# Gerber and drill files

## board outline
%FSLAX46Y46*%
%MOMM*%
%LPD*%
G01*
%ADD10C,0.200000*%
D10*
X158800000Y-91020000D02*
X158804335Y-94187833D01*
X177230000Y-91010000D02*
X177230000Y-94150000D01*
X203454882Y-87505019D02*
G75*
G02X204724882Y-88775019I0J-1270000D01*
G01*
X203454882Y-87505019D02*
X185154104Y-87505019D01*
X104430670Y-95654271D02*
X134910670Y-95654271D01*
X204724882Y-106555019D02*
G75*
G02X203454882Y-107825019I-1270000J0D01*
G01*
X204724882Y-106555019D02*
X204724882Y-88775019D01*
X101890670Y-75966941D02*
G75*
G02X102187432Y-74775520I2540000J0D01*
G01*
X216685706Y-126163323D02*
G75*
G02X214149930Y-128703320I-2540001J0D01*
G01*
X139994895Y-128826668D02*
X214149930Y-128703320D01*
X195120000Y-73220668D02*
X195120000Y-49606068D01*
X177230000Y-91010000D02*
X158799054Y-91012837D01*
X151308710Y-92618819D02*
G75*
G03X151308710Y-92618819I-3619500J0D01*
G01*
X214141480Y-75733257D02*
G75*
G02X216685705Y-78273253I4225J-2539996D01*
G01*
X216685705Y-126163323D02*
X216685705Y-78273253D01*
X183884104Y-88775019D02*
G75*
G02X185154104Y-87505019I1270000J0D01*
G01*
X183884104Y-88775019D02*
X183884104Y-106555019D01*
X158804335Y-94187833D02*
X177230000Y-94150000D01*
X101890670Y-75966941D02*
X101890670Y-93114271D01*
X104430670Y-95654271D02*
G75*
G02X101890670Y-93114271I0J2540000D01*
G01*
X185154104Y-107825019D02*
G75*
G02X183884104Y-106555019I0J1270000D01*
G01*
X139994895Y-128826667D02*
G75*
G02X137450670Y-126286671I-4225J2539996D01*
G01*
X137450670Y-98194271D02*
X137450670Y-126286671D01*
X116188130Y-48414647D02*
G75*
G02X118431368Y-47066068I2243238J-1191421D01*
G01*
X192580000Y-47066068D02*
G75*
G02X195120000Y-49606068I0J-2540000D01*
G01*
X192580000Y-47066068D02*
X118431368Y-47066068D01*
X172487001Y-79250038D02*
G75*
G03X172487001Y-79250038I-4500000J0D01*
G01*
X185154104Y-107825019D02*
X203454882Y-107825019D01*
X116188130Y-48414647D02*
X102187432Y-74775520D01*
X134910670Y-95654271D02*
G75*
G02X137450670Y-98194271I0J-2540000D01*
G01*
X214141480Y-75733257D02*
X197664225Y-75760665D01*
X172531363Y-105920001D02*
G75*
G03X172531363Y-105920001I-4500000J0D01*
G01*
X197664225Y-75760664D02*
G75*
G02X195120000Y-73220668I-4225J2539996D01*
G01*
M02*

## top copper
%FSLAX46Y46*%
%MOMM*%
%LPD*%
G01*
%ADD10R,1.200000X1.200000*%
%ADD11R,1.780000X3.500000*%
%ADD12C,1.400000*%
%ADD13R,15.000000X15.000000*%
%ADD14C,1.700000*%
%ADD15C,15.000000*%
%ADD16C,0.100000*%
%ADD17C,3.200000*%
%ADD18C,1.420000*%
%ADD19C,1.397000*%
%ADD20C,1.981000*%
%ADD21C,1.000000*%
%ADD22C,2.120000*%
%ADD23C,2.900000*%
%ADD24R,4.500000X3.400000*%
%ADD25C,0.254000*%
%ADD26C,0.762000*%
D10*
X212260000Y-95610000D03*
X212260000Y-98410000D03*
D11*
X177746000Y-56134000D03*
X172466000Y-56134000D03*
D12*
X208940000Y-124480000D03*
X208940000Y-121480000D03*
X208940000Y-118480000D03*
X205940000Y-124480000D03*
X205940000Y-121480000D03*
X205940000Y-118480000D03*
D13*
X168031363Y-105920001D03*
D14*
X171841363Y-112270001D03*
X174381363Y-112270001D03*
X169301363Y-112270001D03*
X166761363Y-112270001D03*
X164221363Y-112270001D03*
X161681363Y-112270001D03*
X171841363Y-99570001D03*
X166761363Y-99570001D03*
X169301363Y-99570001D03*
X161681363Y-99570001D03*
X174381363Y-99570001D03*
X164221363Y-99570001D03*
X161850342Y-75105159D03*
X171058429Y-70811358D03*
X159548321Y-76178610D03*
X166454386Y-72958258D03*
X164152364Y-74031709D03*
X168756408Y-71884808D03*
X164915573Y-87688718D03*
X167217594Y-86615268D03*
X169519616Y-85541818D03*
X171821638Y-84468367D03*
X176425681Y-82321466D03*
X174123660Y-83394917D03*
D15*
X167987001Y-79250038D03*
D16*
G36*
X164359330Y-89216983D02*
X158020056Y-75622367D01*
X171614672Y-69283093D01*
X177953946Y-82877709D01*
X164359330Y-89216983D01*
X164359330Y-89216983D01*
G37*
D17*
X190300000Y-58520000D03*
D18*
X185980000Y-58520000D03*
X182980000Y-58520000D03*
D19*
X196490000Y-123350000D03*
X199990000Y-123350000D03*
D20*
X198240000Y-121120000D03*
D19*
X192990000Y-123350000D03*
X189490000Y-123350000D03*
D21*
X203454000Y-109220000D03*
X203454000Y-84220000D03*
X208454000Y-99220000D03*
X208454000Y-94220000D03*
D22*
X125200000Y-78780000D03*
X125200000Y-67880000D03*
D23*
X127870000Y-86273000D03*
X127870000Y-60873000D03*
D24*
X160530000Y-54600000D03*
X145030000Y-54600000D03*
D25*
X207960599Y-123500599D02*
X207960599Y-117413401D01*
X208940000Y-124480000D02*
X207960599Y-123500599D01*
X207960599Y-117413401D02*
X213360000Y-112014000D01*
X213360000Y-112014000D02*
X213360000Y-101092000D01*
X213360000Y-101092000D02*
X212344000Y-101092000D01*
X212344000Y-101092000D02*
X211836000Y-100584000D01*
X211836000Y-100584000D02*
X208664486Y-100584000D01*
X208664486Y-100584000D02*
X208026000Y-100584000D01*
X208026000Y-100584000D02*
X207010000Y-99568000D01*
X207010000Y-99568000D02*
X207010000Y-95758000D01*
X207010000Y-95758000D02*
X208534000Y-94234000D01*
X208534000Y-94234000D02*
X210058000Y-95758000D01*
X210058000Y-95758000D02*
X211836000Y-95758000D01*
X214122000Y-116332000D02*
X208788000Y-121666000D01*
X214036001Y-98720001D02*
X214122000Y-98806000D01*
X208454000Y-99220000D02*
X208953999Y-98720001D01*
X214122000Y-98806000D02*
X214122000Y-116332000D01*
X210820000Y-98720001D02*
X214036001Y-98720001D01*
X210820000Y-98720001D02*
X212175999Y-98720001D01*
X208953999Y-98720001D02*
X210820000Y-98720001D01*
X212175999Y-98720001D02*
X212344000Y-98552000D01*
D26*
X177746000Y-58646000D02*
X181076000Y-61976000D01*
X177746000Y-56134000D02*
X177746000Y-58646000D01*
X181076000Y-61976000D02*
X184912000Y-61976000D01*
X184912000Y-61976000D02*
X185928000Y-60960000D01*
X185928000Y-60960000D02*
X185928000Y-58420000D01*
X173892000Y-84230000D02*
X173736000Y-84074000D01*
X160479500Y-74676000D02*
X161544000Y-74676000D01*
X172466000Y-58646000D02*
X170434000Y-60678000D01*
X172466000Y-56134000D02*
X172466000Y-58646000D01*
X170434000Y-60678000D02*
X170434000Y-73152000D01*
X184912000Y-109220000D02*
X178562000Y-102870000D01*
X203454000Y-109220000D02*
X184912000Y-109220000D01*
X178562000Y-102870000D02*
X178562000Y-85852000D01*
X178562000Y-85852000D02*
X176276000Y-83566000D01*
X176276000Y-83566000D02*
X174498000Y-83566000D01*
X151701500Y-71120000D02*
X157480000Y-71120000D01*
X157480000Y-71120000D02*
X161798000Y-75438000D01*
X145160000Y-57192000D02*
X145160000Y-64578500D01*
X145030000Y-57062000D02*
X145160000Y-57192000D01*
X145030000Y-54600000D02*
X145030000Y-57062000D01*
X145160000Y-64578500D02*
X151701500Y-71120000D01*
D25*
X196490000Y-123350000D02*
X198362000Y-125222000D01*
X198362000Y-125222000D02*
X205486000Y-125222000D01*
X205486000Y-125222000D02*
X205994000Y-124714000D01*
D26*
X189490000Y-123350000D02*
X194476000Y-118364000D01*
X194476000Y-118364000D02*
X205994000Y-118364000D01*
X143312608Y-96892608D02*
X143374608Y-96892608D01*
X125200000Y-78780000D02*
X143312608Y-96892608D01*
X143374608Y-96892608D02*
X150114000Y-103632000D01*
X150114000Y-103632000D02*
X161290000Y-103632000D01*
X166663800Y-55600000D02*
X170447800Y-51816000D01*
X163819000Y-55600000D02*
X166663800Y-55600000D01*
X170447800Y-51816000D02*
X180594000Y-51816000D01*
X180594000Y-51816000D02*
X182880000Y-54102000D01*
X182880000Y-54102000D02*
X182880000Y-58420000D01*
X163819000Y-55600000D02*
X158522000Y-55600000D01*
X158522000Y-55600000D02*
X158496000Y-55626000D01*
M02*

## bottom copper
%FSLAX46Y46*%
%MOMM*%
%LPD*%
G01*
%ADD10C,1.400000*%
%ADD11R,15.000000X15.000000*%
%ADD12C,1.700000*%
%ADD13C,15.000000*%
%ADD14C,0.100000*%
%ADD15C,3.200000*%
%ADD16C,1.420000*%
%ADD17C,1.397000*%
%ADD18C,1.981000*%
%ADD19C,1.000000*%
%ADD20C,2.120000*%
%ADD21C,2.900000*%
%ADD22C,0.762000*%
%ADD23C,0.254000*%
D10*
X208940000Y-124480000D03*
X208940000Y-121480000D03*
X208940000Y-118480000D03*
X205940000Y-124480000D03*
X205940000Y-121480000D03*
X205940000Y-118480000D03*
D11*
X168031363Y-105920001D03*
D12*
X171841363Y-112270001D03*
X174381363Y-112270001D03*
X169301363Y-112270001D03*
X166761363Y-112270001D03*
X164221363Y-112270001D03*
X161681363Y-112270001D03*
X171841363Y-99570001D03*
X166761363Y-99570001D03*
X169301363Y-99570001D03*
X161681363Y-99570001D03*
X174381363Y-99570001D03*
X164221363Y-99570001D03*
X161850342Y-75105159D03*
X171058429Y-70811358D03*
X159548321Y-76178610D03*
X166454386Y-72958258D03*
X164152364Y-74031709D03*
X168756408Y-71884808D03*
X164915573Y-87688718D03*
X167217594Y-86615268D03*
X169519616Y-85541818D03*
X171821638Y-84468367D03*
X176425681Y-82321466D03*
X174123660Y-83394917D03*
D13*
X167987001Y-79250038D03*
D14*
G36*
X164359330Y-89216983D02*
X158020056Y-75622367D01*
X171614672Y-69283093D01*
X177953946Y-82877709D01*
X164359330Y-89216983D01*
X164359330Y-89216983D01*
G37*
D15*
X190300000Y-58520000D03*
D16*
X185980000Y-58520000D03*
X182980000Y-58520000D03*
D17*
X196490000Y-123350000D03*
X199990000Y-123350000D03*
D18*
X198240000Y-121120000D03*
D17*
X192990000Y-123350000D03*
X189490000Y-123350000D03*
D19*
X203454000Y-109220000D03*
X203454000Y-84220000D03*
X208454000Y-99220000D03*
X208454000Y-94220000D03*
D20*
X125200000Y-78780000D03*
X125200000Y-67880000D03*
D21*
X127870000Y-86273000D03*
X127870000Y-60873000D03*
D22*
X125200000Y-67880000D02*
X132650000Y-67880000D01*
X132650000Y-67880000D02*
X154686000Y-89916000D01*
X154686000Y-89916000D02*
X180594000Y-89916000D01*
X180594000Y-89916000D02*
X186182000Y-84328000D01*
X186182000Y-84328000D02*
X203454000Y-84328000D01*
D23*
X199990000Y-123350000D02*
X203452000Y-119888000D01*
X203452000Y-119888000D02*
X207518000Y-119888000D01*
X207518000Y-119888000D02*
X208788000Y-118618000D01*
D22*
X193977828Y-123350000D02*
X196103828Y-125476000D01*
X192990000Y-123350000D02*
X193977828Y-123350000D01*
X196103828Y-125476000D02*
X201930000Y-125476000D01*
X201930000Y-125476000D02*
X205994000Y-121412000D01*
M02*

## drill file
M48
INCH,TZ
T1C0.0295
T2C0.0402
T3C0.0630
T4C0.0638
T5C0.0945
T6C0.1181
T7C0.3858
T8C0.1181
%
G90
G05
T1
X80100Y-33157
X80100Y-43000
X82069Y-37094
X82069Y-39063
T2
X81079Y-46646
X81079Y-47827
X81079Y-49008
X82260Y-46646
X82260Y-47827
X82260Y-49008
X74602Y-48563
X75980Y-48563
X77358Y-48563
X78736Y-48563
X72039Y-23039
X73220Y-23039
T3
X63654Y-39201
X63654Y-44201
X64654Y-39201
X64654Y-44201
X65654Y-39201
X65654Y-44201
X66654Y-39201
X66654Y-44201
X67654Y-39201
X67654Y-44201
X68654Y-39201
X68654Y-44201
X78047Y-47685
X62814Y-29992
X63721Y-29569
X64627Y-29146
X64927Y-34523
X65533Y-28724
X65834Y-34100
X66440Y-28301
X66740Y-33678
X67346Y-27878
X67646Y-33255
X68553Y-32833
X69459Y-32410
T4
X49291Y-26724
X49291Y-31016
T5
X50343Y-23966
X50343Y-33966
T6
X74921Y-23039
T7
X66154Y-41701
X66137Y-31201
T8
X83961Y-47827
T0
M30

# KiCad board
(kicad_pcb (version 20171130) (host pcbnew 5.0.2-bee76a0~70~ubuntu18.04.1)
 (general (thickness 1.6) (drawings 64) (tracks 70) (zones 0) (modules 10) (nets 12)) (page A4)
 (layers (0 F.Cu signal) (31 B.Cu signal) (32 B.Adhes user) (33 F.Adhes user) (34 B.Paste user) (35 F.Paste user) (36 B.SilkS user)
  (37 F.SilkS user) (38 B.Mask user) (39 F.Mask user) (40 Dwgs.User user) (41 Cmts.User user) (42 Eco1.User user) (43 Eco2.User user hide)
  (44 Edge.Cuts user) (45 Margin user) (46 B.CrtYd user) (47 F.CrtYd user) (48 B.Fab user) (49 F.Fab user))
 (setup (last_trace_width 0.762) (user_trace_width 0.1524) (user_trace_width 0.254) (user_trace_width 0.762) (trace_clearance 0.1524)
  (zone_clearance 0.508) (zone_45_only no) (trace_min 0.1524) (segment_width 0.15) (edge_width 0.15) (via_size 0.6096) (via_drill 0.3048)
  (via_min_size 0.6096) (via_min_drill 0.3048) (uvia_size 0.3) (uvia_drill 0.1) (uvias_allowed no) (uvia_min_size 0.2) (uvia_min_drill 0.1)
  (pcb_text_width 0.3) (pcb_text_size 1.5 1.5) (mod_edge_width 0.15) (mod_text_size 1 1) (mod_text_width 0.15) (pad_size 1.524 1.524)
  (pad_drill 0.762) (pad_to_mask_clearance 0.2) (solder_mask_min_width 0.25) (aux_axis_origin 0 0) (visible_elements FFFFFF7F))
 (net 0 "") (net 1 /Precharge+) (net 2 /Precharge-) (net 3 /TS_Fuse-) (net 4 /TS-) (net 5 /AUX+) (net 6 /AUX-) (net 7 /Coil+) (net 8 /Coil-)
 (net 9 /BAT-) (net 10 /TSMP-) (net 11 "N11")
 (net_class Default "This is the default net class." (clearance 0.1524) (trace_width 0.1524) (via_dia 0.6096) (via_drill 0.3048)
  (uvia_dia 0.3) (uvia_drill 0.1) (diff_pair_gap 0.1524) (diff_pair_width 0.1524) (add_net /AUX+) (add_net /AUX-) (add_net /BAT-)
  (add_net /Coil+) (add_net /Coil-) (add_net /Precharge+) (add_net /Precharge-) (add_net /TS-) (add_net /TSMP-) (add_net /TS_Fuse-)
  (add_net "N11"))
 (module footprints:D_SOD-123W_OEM (layer F.Cu) (at 212.26 97.01 270)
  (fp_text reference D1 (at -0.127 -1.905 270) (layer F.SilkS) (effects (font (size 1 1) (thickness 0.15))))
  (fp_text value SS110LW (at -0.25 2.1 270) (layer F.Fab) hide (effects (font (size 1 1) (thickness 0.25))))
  (pad 1 smd rect (at -1.4 0 270) (size 1.2 1.2) (layers F.Cu F.Paste F.Mask) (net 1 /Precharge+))
  (pad 2 smd rect (at 1.4 0 270) (size 1.2 1.2) (layers F.Cu F.Paste F.Mask) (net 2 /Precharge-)))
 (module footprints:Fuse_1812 (layer F.Cu) (at 172.466 56.134)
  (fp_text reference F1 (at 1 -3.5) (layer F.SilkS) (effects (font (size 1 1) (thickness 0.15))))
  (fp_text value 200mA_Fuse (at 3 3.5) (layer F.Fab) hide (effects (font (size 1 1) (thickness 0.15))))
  (pad 2 smd rect (at 5.28 0) (size 1.78 3.5) (layers F.Cu F.Paste F.Mask) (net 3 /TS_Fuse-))
  (pad 1 smd rect (at 0 0) (size 1.78 3.5) (layers F.Cu F.Paste F.Mask) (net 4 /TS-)))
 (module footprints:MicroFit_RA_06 (layer B.Cu) (at 213.26 121.48 90)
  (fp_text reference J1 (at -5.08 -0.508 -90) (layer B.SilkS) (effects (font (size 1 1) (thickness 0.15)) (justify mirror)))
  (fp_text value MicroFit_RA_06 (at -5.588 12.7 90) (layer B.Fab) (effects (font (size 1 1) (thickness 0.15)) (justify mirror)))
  (pad "" np_thru_hole circle (at 0 0 270) (size 3 3) (drill 3) (layers *.Cu *.Mask))
  (pad 1 thru_hole circle (at -3 -4.32 270) (size 1.4 1.4) (drill 1.02) (layers *.Cu *.Mask) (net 1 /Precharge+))
  (pad 2 thru_hole circle (at 0 -4.32 270) (size 1.4 1.4) (drill 1.02) (layers *.Cu *.Mask) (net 2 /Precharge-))
  (pad 3 thru_hole circle (at 3 -4.32 270) (size 1.4 1.4) (drill 1.02) (layers *.Cu *.Mask) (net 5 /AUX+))
  (pad 4 thru_hole circle (at -3 -7.32 270) (size 1.4 1.4) (drill 1.02) (layers *.Cu *.Mask) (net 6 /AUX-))
  (pad 5 thru_hole circle (at 0 -7.32 270) (size 1.4 1.4) (drill 1.02) (layers *.Cu *.Mask) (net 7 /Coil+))
  (pad 6 thru_hole circle (at 3 -7.32 270) (size 1.4 1.4) (drill 1.02) (layers *.Cu *.Mask) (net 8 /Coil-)))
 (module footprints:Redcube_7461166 (layer F.Cu) (at 168.031363 105.920001)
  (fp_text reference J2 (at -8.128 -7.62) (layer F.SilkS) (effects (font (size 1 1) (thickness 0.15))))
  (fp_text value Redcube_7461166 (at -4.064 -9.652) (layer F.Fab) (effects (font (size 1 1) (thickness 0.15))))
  (pad 1 thru_hole rect (at 0 0) (size 15 15) (drill 9.8) (layers *.Cu *.Mask) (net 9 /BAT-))
  (pad 1 thru_hole circle (at 3.81 6.35) (size 1.7 1.7) (drill 1.6) (layers *.Cu *.Mask) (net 9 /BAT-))
  (pad 1 thru_hole circle (at 6.35 6.35) (size 1.7 1.7) (drill 1.6) (layers *.Cu *.Mask) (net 9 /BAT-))
  (pad 1 thru_hole circle (at 1.27 6.35) (size 1.7 1.7) (drill 1.6) (layers *.Cu *.Mask) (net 9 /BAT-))
  (pad 1 thru_hole circle (at -1.27 6.35) (size 1.7 1.7) (drill 1.6) (layers *.Cu *.Mask) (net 9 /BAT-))
  (pad 1 thru_hole circle (at -3.81 6.35) (size 1.7 1.7) (drill 1.6) (layers *.Cu *.Mask) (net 9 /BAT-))
  (pad 1 thru_hole circle (at -6.35 6.35) (size 1.7 1.7) (drill 1.6) (layers *.Cu *.Mask) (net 9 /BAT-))
  (pad 1 thru_hole circle (at 3.81 -6.35) (size 1.7 1.7) (drill 1.6) (layers *.Cu *.Mask) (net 9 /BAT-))
  (pad 1 thru_hole circle (at -1.27 -6.35) (size 1.7 1.7) (drill 1.6) (layers *.Cu *.Mask) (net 9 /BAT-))
  (pad 1 thru_hole circle (at 1.27 -6.35) (size 1.7 1.7) (drill 1.6) (layers *.Cu *.Mask) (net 9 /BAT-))
  (pad 1 thru_hole circle (at -6.35 -6.35) (size 1.7 1.7) (drill 1.6) (layers *.Cu *.Mask) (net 9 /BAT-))
  (pad 1 thru_hole circle (at 6.35 -6.35) (size 1.7 1.7) (drill 1.6) (layers *.Cu *.Mask) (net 9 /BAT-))
  (pad 1 thru_hole circle (at -3.81 -6.35) (size 1.7 1.7) (drill 1.6) (layers *.Cu *.Mask) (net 9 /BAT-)))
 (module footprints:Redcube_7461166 (layer F.Cu) (at 167.987001 79.250038 25)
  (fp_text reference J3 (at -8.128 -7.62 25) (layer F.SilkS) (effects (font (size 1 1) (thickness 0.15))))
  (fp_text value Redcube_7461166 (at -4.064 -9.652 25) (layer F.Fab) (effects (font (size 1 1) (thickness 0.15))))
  (pad 1 thru_hole circle (at -3.81 -6.35 25) (size 1.7 1.7) (drill 1.6) (layers *.Cu *.Mask) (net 4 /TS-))
  (pad 1 thru_hole circle (at 6.349999 -6.35 25) (size 1.7 1.7) (drill 1.6) (layers *.Cu *.Mask) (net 4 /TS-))
  (pad 1 thru_hole circle (at -6.35 -6.349999 25) (size 1.7 1.7) (drill 1.6) (layers *.Cu *.Mask) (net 4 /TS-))
  (pad 1 thru_hole circle (at 1.27 -6.35 25) (size 1.7 1.7) (drill 1.6) (layers *.Cu *.Mask) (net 4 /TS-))
  (pad 1 thru_hole circle (at -1.27 -6.35 25) (size 1.7 1.7) (drill 1.6) (layers *.Cu *.Mask) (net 4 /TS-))
  (pad 1 thru_hole circle (at 3.81 -6.35 25) (size 1.7 1.7) (drill 1.6) (layers *.Cu *.Mask) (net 4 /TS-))
  (pad 1 thru_hole circle (at -6.349999 6.35 25) (size 1.7 1.7) (drill 1.6) (layers *.Cu *.Mask) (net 4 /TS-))
  (pad 1 thru_hole circle (at -3.81 6.35 25) (size 1.7 1.7) (drill 1.6) (layers *.Cu *.Mask) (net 4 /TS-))
  (pad 1 thru_hole circle (at -1.27 6.35 25) (size 1.7 1.7) (drill 1.6) (layers *.Cu *.Mask) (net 4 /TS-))
  (pad 1 thru_hole circle (at 1.27 6.35 25) (size 1.7 1.7) (drill 1.6) (layers *.Cu *.Mask) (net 4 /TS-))
  (pad 1 thru_hole circle (at 6.35 6.349999 25) (size 1.7 1.7) (drill 1.6) (layers *.Cu *.Mask) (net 4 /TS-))
  (pad 1 thru_hole circle (at 3.81 6.35 25) (size 1.7 1.7) (drill 1.6) (layers *.Cu *.Mask) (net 4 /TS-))
  (pad 1 thru_hole rect (at 0 0 25) (size 15 15) (drill 9.8) (layers *.Cu *.Mask) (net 4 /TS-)))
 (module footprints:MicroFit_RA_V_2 (layer B.Cu) (at 190.3 58.52 90)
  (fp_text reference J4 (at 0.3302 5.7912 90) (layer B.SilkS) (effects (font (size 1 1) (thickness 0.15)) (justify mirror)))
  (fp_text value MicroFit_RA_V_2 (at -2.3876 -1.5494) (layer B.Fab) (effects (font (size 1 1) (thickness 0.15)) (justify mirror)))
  (pad "" thru_hole circle (at 0 0 90) (size 3.2 3.2) (drill 3) (layers *.Cu *.Mask))
  (pad 1 thru_hole circle (at 0 -4.32 90) (size 1.42 1.42) (drill 1.02) (layers *.Cu *.Mask) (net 3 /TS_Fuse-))
  (pad 2 thru_hole circle (at 0 -7.32 90) (size 1.42 1.42) (drill 1.02) (layers *.Cu *.Mask) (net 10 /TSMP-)))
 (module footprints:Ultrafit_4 (layer F.Cu) (at 194.74 123.35 90)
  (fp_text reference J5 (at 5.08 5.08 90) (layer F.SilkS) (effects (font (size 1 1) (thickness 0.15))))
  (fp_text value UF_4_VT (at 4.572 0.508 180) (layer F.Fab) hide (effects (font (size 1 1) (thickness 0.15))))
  (pad 2 thru_hole circle (at 0 1.75 90) (size 1.397 1.397) (drill 1.02) (layers *.Cu *.Mask) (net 6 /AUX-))
  (pad 1 thru_hole circle (at 0 5.25 90) (size 1.397 1.397) (drill 1.02) (layers *.Cu *.Mask) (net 5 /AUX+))
  (pad "" thru_hole circle (at 2.23 3.5 90) (size 1.981 1.981) (drill 1.6) (layers *.Cu *.Mask))
  (pad 3 thru_hole circle (at 0 -1.75 270) (size 1.397 1.397) (drill 1.02) (layers *.Cu *.Mask) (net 7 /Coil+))
  (pad 4 thru_hole circle (at 0 -5.25 270) (size 1.397 1.397) (drill 1.02) (layers *.Cu *.Mask) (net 8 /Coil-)))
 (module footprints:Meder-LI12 (layer B.Cu) (at 203.454 109.22 90)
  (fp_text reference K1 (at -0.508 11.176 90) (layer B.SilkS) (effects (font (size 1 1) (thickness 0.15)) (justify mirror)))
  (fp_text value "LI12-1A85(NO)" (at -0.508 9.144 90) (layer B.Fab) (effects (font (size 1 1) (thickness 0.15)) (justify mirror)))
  (pad 1 thru_hole circle (at 0 0 90) (size 1 1) (drill 0.75) (layers *.Cu *.Mask) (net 4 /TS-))
  (pad 2 thru_hole circle (at 25 0 90) (size 1 1) (drill 0.75) (layers *.Cu *.Mask) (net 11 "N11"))
  (pad 3 thru_hole circle (at 10 5 90) (size 1 1) (drill 0.75) (layers *.Cu *.Mask) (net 2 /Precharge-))
  (pad 4 thru_hole circle (at 15 5 90) (size 1 1) (drill 0.75) (layers *.Cu *.Mask) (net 1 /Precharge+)))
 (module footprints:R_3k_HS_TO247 (layer B.Cu) (at 125.2 78.78 90)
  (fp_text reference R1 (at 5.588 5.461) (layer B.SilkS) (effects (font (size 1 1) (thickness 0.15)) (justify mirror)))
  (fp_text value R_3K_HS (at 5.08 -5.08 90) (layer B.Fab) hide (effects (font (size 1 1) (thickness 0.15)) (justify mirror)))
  (pad 1 thru_hole circle (at 0 0 90) (size 2.12 2.12) (drill 1.62) (layers *.Cu *.Mask) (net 9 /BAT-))
  (pad 2 thru_hole circle (at 10.9 0 90) (size 2.12 2.12) (drill 1.62) (layers *.Cu *.Mask) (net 11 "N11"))
  (pad 4 thru_hole circle (at -7.493 2.67 90) (size 2.9 2.9) (drill 2.4) (layers *.Cu *.Mask))
  (pad 5 thru_hole circle (at 17.907 2.67 90) (size 2.9 2.9) (drill 2.4) (layers *.Cu *.Mask)))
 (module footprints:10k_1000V (layer F.Cu) (at 160.53 54.6 180)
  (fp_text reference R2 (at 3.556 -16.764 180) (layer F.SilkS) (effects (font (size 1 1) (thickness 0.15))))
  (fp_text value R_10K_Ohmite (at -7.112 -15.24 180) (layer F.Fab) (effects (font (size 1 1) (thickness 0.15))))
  (pad 1 smd rect (at 0 0 180) (size 4.5 3.4) (layers F.Cu F.Paste F.Mask) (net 10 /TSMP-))
  (pad 2 smd rect (at 15.5 0 180) (size 4.5 3.4) (layers F.Cu F.Paste F.Mask) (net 4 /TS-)))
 (gr_line (start 158.8 91.02) (end 158.804335 94.187833) (layer Edge.Cuts) (width 0.2))
 (gr_line (start 177.23 91.01) (end 177.23 94.15) (layer Edge.Cuts) (width 0.2))
 (gr_arc (start 203.454882 88.775019) (end 204.724882 88.775019) (angle -90) (layer Edge.Cuts) (width 0.2))
 (gr_line (start 203.454882 87.505019) (end 185.154104 87.505019) (layer Edge.Cuts) (width 0.2))
 (gr_line (start 104.43067 95.654271) (end 134.91067 95.654271) (layer Edge.Cuts) (width 0.2))
 (gr_arc (start 203.454882 106.555019) (end 203.454882 107.825019) (angle -90) (layer Edge.Cuts) (width 0.2))
 (gr_line (start 204.724882 106.555019) (end 204.724882 88.775019) (layer Edge.Cuts) (width 0.2))
 (gr_arc (start 104.43067 75.966941) (end 102.187432 74.77552) (angle -27.9735142) (layer Edge.Cuts) (width 0.2))
 (gr_arc (start 214.145705 126.163323) (end 214.14993 128.70332) (angle -89.90469527) (layer Edge.Cuts) (width 0.2))
 (gr_line (start 139.994895 128.826668) (end 214.14993 128.70332) (layer Edge.Cuts) (width 0.2))
 (gr_line (start 195.12 73.220668) (end 195.12 49.606068) (layer Edge.Cuts) (width 0.2))
 (gr_line (start 177.23 91.01) (end 158.799054 91.012837) (layer Edge.Cuts) (width 0.2))
 (gr_circle (center 147.68921 92.618819) (end 151.30871 92.618819) (layer Edge.Cuts) (width 0.2))
 (gr_arc (start 214.145705 78.273253) (end 216.685705 78.273253) (angle -90.09530473) (layer Edge.Cuts) (width 0.2))
 (gr_line (start 216.685705 126.163323) (end 216.685705 78.273253) (layer Edge.Cuts) (width 0.2))
 (gr_arc (start 185.154104 88.775019) (end 185.154104 87.505019) (angle -90) (layer Edge.Cuts) (width 0.2))
 (gr_line (start 183.884104 88.775019) (end 183.884104 106.555019) (layer Edge.Cuts) (width 0.2))
 (gr_line (start 158.804335 94.187833) (end 177.23 94.15) (layer Edge.Cuts) (width 0.2))
 (gr_line (start 101.89067 75.966941) (end 101.89067 93.114271) (layer Edge.Cuts) (width 0.2))
 (gr_arc (start 104.43067 93.114271) (end 101.89067 93.114271) (angle -90) (layer Edge.Cuts) (width 0.2))
 (gr_arc (start 185.154104 106.555019) (end 183.884104 106.555019) (angle -90) (layer Edge.Cuts) (width 0.2))
 (gr_arc (start 139.99067 126.286671) (end 137.45067 126.286671) (angle -90.09530473) (layer Edge.Cuts) (width 0.2))
 (gr_line (start 137.45067 98.194271) (end 137.45067 126.286671) (layer Edge.Cuts) (width 0.2))
 (gr_arc (start 118.431368 49.606068) (end 118.431368 47.066068) (angle -62.0264858) (layer Edge.Cuts) (width 0.2))
 (gr_arc (start 192.58 49.606068) (end 195.12 49.606068) (angle -90) (layer Edge.Cuts) (width 0.2))
 (gr_line (start 192.58 47.066068) (end 118.431368 47.066068) (layer Edge.Cuts) (width 0.2))
 (gr_circle (center 167.987001 79.250038) (end 172.487001 79.250038) (layer Edge.Cuts) (width 0.2))
 (gr_line (start 185.154104 107.825019) (end 203.454882 107.825019) (layer Edge.Cuts) (width 0.2))
 (gr_line (start 116.18813 48.414647) (end 102.187432 74.77552) (layer Edge.Cuts) (width 0.2))
 (gr_arc (start 134.91067 98.194271) (end 137.45067 98.194271) (angle -90) (layer Edge.Cuts) (width 0.2))
 (gr_line (start 214.14148 75.733257) (end 197.664225 75.760665) (layer Edge.Cuts) (width 0.2))
 (gr_circle (center 168.031363 105.920001) (end 172.531363 105.920001) (layer Edge.Cuts) (width 0.2))
 (gr_arc (start 197.66 73.220668) (end 195.12 73.220668) (angle -90.09530473) (layer Edge.Cuts) (width 0.2))
 (segment (start 125.2 67.88) (end 132.65 67.88) (width 0.762) (layer B.Cu) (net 11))
 (segment (start 132.65 67.88) (end 154.686 89.916) (width 0.762) (layer B.Cu) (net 11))
 (segment (start 154.686 89.916) (end 180.594 89.916) (width 0.762) (layer B.Cu) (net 11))
 (segment (start 180.594 89.916) (end 186.182 84.328) (width 0.762) (layer B.Cu) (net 11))
 (segment (start 186.182 84.328) (end 203.454 84.328) (width 0.762) (layer B.Cu) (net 11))
 (segment (start 207.960599 123.500599) (end 207.960599 117.413401) (width 0.254) (layer F.Cu) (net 1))
 (segment (start 208.94 124.48) (end 207.960599 123.500599) (width 0.254) (layer F.Cu) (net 1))
 (segment (start 207.960599 117.413401) (end 213.36 112.014) (width 0.254) (layer F.Cu) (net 1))
 (segment (start 213.36 112.014) (end 213.36 101.092) (width 0.254) (layer F.Cu) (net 1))
 (segment (start 213.36 101.092) (end 212.344 101.092) (width 0.254) (layer F.Cu) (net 1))
 (segment (start 212.344 101.092) (end 211.836 100.584) (width 0.254) (layer F.Cu) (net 1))
 (segment (start 211.836 100.584) (end 208.664486 100.584) (width 0.254) (layer F.Cu) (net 1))
 (segment (start 208.664486 100.584) (end 208.026 100.584) (width 0.254) (layer F.Cu) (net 1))
 (segment (start 208.026 100.584) (end 207.01 99.568) (width 0.254) (layer F.Cu) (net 1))
 (segment (start 207.01 99.568) (end 207.01 95.758) (width 0.254) (layer F.Cu) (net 1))
 (segment (start 207.01 95.758) (end 208.534 94.234) (width 0.254) (layer F.Cu) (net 1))
 (segment (start 208.534 94.234) (end 210.058 95.758) (width 0.254) (layer F.Cu) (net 1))
 (segment (start 210.058 95.758) (end 211.836 95.758) (width 0.254) (layer F.Cu) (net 1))
 (segment (start 214.122 116.332) (end 208.788 121.666) (width 0.254) (layer F.Cu) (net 2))
 (segment (start 214.036001 98.720001) (end 214.122 98.806) (width 0.254) (layer F.Cu) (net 2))
 (segment (start 208.454 99.22) (end 208.953999 98.720001) (width 0.254) (layer F.Cu) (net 2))
 (segment (start 214.122 98.806) (end 214.122 116.332) (width 0.254) (layer F.Cu) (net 2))
 (segment (start 210.82 98.720001) (end 214.036001 98.720001) (width 0.254) (layer F.Cu) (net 2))
 (segment (start 210.82 98.720001) (end 212.175999 98.720001) (width 0.254) (layer F.Cu) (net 2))
 (segment (start 208.953999 98.720001) (end 210.82 98.720001) (width 0.254) (layer F.Cu) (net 2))
 (segment (start 212.175999 98.720001) (end 212.344 98.552) (width 0.254) (layer F.Cu) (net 2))
 (segment (start 177.746 58.646) (end 181.076 61.976) (width 0.762) (layer F.Cu) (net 3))
 (segment (start 177.746 56.134) (end 177.746 58.646) (width 0.762) (layer F.Cu) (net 3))
 (segment (start 181.076 61.976) (end 184.912 61.976) (width 0.762) (layer F.Cu) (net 3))
 (segment (start 184.912 61.976) (end 185.928 60.96) (width 0.762) (layer F.Cu) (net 3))
 (segment (start 185.928 60.96) (end 185.928 58.42) (width 0.762) (layer F.Cu) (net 3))
 (segment (start 173.892 84.23) (end 173.736 84.074) (width 0.762) (layer F.Cu) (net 4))
 (segment (start 160.4795 74.676) (end 161.544 74.676) (width 0.762) (layer F.Cu) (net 4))
 (segment (start 172.466 58.646) (end 170.434 60.678) (width 0.762) (layer F.Cu) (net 4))
 (segment (start 172.466 56.134) (end 172.466 58.646) (width 0.762) (layer F.Cu) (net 4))
 (segment (start 170.434 60.678) (end 170.434 73.152) (width 0.762) (layer F.Cu) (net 4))
 (segment (start 184.912 109.22) (end 178.562 102.87) (width 0.762) (layer F.Cu) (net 4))
 (segment (start 203.454 109.22) (end 184.912 109.22) (width 0.762) (layer F.Cu) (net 4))
 (segment (start 178.562 102.87) (end 178.562 85.852) (width 0.762) (layer F.Cu) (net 4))
 (segment (start 178.562 85.852) (end 176.276 83.566) (width 0.762) (layer F.Cu) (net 4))
 (segment (start 176.276 83.566) (end 174.498 83.566) (width 0.762) (layer F.Cu) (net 4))
 (segment (start 151.7015 71.12) (end 157.48 71.12) (width 0.762) (layer F.Cu) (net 4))
 (segment (start 157.48 71.12) (end 161.798 75.438) (width 0.762) (layer F.Cu) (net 4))
 (segment (start 145.16 57.192) (end 145.16 64.5785) (width 0.762) (layer F.Cu) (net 4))
 (segment (start 145.03 57.062) (end 145.16 57.192) (width 0.762) (layer F.Cu) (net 4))
 (segment (start 145.03 54.6) (end 145.03 57.062) (width 0.762) (layer F.Cu) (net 4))
 (segment (start 145.16 64.5785) (end 151.7015 71.12) (width 0.762) (layer F.Cu) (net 4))
 (segment (start 199.99 123.35) (end 203.452 119.888) (width 0.254) (layer B.Cu) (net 5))
 (segment (start 203.452 119.888) (end 207.518 119.888) (width 0.254) (layer B.Cu) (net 5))
 (segment (start 207.518 119.888) (end 208.788 118.618) (width 0.254) (layer B.Cu) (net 5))
 (segment (start 196.49 123.35) (end 198.362 125.222) (width 0.254) (layer F.Cu) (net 6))
 (segment (start 198.362 125.222) (end 205.486 125.222) (width 0.254) (layer F.Cu) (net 6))
 (segment (start 205.486 125.222) (end 205.994 124.714) (width 0.254) (layer F.Cu) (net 6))
 (segment (start 193.977828 123.35) (end 196.103828 125.476) (width 0.762) (layer B.Cu) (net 7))
 (segment (start 192.99 123.35) (end 193.977828 123.35) (width 0.762) (layer B.Cu) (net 7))
 (segment (start 196.103828 125.476) (end 201.93 125.476) (width 0.762) (layer B.Cu) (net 7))
 (segment (start 201.93 125.476) (end 205.994 121.412) (width 0.762) (layer B.Cu) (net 7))
 (segment (start 189.49 123.35) (end 194.476 118.364) (width 0.762) (layer F.Cu) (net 8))
 (segment (start 194.476 118.364) (end 205.994 118.364) (width 0.762) (layer F.Cu) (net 8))
 (segment (start 143.312608 96.892608) (end 143.374608 96.892608) (width 0.762) (layer F.Cu) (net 9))
 (segment (start 125.2 78.78) (end 143.312608 96.892608) (width 0.762) (layer F.Cu) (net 9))
 (segment (start 143.374608 96.892608) (end 150.114 103.632) (width 0.762) (layer F.Cu) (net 9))
 (segment (start 150.114 103.632) (end 161.29 103.632) (width 0.762) (layer F.Cu) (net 9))
 (segment (start 166.6638 55.6) (end 170.4478 51.816) (width 0.762) (layer F.Cu) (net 10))
 (segment (start 163.819 55.6) (end 166.6638 55.6) (width 0.762) (layer F.Cu) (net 10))
 (segment (start 170.4478 51.816) (end 180.594 51.816) (width 0.762) (layer F.Cu) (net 10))
 (segment (start 180.594 51.816) (end 182.88 54.102) (width 0.762) (layer F.Cu) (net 10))
 (segment (start 182.88 54.102) (end 182.88 58.42) (width 0.762) (layer F.Cu) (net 10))
 (segment (start 163.819 55.6) (end 158.522 55.6) (width 0.762) (layer F.Cu) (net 10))
 (segment (start 158.522 55.6) (end 158.496 55.626) (width 0.762) (layer F.Cu) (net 10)))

